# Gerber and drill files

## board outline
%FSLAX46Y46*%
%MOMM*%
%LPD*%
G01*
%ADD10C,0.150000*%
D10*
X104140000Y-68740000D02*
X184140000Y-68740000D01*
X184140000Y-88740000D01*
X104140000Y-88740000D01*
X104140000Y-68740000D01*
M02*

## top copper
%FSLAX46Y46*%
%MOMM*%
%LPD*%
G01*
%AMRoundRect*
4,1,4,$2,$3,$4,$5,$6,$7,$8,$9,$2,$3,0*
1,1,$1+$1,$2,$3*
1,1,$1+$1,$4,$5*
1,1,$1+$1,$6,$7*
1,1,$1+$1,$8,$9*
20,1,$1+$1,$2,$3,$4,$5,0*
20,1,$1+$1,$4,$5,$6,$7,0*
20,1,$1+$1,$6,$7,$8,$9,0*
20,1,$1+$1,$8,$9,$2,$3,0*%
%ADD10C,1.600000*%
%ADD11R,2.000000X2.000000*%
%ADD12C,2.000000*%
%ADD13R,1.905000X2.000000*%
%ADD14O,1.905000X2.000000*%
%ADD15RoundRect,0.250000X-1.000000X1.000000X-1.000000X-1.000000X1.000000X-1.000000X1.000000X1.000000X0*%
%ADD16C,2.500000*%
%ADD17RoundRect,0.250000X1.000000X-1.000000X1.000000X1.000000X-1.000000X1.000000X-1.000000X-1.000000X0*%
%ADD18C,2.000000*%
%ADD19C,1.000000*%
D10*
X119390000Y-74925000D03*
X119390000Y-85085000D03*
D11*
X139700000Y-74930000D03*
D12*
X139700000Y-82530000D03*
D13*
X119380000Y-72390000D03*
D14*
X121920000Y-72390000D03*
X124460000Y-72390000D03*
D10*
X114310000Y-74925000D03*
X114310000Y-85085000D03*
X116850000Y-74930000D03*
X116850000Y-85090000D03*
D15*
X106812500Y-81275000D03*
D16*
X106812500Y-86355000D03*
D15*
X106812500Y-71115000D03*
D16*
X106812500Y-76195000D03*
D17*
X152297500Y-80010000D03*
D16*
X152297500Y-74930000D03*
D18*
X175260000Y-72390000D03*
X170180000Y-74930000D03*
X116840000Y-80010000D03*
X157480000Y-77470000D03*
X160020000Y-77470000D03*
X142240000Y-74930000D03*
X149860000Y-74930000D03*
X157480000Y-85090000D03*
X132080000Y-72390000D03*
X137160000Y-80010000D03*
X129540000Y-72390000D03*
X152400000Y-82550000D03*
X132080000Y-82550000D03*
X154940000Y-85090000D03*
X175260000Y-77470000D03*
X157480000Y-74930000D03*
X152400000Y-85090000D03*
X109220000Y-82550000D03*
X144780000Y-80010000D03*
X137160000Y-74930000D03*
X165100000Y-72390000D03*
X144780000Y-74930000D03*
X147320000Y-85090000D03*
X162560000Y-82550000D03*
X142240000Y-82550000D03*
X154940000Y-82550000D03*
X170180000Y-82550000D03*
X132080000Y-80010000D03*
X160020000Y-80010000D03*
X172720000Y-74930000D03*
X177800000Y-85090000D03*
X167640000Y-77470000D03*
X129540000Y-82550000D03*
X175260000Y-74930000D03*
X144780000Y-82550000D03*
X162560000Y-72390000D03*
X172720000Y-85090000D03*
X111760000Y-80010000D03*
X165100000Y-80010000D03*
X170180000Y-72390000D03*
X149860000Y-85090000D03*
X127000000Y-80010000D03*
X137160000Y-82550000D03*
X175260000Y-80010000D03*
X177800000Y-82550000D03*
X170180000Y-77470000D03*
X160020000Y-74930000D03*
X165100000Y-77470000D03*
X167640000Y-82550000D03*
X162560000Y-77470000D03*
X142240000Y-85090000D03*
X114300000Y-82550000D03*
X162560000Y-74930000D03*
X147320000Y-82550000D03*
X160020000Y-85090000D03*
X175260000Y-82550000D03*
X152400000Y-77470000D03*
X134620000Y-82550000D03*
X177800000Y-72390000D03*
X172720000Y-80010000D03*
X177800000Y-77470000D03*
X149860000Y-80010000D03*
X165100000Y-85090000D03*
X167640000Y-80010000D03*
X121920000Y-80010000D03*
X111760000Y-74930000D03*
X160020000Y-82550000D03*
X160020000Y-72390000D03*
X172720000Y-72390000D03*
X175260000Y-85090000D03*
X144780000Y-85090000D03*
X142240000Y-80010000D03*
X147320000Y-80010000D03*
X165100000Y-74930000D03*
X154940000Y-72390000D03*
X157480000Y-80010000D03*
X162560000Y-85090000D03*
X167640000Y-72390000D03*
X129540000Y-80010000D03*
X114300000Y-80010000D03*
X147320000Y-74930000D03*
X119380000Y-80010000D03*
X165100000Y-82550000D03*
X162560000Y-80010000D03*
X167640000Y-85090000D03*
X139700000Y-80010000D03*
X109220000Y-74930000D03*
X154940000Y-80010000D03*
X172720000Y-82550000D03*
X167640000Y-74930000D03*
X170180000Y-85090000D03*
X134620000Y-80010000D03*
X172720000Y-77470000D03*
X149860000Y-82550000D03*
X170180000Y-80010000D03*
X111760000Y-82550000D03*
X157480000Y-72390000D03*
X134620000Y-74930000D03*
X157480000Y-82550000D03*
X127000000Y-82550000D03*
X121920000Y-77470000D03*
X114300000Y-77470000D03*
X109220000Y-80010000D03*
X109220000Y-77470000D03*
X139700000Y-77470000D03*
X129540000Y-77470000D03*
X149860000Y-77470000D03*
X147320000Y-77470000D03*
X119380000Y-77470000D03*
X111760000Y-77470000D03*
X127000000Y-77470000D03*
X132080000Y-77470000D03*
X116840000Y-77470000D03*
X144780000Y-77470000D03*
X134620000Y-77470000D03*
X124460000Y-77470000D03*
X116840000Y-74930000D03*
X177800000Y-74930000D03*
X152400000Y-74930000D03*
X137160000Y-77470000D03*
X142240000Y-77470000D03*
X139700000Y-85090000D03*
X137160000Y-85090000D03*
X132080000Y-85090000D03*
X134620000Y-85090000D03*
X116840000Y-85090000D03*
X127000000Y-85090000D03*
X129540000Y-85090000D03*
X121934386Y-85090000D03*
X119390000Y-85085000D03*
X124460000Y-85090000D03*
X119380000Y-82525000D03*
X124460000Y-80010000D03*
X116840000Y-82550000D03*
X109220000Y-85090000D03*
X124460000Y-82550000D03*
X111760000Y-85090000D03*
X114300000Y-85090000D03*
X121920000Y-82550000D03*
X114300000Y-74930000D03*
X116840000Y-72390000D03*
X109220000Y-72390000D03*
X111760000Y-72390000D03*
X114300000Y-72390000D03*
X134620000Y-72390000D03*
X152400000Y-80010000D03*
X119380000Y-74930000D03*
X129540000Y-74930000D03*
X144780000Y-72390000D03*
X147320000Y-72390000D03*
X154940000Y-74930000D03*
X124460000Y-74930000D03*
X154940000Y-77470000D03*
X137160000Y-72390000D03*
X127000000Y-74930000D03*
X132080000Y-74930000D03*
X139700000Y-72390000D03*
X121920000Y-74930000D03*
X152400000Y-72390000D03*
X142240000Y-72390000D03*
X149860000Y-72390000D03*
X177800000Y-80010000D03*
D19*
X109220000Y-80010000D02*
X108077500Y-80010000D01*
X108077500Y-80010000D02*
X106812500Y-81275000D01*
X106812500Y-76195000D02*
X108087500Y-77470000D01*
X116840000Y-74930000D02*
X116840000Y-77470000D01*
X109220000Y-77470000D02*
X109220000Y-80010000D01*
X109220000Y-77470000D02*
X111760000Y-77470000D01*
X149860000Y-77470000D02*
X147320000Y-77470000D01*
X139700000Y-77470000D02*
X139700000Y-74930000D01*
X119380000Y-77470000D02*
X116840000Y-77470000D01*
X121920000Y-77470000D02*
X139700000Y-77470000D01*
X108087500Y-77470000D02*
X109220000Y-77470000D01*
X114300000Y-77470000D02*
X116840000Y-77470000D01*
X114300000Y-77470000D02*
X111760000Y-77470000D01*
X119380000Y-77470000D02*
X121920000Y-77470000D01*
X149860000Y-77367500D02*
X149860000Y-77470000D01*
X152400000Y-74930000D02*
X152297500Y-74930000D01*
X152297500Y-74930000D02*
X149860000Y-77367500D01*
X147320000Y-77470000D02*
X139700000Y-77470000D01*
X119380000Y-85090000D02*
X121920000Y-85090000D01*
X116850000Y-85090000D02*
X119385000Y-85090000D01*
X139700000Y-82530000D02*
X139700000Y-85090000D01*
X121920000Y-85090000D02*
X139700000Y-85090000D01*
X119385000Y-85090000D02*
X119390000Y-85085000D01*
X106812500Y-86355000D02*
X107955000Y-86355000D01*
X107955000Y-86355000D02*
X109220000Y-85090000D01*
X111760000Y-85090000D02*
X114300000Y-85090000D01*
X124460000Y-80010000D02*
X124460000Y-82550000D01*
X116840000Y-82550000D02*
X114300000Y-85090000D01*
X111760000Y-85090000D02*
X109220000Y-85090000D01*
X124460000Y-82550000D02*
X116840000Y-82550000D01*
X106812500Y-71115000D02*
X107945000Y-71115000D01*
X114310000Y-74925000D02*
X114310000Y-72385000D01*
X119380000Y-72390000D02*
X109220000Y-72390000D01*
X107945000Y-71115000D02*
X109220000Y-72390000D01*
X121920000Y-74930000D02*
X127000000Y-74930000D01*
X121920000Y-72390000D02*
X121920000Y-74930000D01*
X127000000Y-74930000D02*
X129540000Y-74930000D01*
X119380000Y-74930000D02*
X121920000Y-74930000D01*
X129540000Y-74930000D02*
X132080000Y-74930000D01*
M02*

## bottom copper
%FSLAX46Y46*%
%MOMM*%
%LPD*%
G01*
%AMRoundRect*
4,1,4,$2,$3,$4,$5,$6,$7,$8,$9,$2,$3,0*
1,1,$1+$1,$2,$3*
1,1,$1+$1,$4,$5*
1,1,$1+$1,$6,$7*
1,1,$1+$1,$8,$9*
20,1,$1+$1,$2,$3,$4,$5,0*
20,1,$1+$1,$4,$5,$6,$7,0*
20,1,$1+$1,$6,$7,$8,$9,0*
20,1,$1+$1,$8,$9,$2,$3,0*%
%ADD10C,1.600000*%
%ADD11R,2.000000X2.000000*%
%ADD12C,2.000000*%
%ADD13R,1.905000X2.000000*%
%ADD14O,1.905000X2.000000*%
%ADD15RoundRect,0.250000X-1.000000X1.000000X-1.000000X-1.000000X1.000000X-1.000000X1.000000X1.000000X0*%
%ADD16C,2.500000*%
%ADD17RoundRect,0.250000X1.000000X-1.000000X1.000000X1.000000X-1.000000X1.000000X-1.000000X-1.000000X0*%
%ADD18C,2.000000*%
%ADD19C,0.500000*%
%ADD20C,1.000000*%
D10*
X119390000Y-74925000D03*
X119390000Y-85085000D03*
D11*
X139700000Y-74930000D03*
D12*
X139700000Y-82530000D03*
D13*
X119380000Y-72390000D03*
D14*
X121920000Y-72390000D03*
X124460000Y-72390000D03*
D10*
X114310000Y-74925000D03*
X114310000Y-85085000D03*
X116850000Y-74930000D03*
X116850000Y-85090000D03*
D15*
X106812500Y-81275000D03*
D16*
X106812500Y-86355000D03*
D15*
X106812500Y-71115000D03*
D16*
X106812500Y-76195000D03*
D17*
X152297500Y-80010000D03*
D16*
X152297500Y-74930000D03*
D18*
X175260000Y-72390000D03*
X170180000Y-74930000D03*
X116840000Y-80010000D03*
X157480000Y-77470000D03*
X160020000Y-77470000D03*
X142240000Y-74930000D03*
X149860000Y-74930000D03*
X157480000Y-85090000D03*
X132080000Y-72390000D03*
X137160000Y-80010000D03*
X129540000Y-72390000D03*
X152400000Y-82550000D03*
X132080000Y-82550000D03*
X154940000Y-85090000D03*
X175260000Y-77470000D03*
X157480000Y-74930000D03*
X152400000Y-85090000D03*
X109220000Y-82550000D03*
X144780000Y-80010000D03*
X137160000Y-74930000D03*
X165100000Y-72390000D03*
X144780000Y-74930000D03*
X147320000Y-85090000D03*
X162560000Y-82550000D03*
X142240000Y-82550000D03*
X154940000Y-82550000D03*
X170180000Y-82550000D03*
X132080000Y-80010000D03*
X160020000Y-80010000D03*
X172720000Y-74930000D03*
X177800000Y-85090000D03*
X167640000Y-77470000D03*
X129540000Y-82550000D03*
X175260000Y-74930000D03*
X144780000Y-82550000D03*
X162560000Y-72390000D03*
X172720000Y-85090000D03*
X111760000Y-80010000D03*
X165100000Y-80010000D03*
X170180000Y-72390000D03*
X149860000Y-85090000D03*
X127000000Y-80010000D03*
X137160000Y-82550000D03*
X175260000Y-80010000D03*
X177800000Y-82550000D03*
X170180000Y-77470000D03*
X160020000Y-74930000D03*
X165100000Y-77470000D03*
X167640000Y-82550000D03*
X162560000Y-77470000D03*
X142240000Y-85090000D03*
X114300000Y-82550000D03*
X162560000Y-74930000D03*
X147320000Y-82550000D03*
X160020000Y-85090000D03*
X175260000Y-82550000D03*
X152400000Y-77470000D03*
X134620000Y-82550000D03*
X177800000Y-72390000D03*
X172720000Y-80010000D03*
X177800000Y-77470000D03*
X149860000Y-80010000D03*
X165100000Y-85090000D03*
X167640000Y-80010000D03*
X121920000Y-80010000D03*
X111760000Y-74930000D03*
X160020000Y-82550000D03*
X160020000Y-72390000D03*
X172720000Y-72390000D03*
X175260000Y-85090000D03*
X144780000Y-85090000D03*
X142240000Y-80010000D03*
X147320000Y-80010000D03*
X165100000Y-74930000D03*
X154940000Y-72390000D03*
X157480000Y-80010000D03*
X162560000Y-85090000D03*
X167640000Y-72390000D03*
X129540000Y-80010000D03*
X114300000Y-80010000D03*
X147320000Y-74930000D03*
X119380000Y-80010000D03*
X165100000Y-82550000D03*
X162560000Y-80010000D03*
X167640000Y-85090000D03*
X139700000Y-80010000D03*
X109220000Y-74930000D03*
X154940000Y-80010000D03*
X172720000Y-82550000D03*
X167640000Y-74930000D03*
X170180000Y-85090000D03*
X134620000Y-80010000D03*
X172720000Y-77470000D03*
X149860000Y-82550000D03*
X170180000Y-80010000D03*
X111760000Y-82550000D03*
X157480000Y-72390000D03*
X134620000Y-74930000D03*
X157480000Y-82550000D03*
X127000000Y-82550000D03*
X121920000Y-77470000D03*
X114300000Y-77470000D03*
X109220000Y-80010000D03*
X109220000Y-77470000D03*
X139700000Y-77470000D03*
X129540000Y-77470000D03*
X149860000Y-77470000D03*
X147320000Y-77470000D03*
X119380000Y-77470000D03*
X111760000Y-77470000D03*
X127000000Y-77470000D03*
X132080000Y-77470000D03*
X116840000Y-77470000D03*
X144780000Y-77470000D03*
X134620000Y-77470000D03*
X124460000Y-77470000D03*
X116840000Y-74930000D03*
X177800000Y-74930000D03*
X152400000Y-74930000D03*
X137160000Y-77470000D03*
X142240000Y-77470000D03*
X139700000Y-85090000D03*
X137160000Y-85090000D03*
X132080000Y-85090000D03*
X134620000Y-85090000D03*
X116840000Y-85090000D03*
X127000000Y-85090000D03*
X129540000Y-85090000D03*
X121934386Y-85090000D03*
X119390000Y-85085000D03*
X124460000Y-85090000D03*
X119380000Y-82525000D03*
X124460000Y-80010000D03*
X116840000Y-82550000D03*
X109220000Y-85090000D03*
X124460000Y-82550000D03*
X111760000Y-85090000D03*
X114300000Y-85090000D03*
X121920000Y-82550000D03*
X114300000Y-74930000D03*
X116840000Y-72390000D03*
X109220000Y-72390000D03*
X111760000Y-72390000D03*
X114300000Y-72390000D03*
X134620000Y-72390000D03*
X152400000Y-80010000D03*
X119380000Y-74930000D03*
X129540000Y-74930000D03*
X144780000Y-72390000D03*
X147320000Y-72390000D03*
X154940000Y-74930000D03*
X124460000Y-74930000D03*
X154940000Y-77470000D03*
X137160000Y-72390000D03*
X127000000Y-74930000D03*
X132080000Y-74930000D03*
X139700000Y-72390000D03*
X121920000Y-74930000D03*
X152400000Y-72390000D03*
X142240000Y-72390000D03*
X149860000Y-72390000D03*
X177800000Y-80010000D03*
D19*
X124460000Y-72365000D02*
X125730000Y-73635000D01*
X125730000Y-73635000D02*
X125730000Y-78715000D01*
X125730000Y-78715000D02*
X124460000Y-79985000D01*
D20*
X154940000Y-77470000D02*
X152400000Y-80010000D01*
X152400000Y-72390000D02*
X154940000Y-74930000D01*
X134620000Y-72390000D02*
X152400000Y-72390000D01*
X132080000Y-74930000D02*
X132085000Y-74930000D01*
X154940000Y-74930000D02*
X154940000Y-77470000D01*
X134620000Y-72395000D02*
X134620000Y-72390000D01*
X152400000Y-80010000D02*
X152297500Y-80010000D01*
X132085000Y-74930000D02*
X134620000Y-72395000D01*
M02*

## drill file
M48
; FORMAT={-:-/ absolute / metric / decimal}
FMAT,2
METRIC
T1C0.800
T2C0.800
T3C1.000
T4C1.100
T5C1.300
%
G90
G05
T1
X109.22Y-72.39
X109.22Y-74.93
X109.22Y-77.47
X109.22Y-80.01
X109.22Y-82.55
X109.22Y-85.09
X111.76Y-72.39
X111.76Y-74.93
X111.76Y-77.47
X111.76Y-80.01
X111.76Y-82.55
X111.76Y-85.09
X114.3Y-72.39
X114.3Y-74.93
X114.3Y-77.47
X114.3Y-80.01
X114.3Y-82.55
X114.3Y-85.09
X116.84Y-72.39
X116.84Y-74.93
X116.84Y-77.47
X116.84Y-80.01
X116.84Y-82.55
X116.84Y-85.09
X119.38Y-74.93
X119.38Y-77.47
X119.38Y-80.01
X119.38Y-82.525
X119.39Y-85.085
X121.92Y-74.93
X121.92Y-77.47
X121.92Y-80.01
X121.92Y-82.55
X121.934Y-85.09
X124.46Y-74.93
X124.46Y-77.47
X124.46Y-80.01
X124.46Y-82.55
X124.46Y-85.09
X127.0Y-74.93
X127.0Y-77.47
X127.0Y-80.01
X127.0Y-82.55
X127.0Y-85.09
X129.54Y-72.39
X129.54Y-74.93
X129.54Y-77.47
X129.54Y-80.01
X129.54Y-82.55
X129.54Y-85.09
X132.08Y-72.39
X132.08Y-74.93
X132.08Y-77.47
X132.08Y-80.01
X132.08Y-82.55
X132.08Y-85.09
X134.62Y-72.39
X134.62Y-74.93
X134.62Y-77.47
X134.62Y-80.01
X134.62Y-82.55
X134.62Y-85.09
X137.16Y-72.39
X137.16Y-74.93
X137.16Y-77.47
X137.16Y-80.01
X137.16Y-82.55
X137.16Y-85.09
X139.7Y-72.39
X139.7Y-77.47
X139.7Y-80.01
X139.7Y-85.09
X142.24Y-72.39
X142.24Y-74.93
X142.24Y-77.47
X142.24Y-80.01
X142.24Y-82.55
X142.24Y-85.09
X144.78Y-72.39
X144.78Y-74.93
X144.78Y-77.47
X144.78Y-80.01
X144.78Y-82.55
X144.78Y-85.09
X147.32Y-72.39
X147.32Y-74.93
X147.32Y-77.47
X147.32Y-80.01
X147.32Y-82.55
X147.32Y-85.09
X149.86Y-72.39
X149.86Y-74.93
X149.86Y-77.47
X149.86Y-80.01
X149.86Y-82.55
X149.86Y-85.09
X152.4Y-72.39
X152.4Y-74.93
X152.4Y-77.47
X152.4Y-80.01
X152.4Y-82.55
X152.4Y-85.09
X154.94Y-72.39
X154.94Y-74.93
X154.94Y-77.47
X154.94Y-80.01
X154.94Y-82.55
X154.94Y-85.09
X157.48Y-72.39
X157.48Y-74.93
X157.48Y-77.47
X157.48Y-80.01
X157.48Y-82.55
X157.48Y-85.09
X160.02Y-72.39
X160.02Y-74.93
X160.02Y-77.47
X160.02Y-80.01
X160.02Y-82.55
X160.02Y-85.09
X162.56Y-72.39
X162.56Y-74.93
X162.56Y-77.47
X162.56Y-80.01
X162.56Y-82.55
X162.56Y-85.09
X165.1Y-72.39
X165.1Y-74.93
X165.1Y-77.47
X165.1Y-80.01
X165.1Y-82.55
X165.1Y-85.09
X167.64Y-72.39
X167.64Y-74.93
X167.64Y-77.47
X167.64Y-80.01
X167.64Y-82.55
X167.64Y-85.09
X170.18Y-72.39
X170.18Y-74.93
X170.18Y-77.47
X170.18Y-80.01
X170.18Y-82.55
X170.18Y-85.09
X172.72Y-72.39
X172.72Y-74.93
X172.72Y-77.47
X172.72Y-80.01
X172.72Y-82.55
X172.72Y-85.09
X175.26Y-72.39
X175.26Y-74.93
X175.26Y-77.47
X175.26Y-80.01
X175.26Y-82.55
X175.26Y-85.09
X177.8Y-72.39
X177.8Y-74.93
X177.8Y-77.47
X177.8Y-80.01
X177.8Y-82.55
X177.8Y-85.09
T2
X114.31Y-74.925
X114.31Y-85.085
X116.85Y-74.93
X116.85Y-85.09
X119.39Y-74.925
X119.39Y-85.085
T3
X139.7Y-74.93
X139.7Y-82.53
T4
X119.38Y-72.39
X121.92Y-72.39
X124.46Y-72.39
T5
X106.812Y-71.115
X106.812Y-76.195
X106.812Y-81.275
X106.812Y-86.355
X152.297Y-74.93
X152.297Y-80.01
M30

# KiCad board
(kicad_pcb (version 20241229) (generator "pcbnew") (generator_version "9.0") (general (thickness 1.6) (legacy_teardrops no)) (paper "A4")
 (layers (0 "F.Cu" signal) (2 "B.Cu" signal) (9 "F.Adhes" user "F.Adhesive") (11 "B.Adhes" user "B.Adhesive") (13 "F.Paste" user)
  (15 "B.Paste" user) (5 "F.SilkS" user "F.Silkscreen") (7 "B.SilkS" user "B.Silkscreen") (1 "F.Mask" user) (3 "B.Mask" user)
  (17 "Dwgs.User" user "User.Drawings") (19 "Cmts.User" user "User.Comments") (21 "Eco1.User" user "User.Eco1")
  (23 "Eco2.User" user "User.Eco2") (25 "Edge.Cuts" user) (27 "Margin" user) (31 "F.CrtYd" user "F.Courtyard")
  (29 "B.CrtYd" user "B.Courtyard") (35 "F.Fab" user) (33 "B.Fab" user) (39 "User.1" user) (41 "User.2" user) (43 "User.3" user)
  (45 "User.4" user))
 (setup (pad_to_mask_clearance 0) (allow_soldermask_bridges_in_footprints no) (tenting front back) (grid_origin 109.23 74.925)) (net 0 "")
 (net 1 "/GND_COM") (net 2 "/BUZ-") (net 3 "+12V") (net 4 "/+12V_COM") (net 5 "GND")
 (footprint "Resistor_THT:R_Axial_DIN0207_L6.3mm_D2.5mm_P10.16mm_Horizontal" (layer "F.Cu") (at 119.39 74.925 -90)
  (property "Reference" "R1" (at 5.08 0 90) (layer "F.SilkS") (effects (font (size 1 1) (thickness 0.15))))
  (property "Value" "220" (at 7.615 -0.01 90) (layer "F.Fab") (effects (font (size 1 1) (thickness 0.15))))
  (pad "1" thru_hole circle (at 0 0 270) (size 1.6 1.6) (drill 0.8) (layers "*.Cu" "*.Mask") (remove_unused_layers no) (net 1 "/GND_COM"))
  (pad "2" thru_hole circle (at 10.16 0 270) (size 1.6 1.6) (drill 0.8) (layers "*.Cu" "*.Mask") (remove_unused_layers no) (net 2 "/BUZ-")))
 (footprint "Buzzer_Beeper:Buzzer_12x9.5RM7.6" (layer "F.Cu") (at 139.7 74.93 -90)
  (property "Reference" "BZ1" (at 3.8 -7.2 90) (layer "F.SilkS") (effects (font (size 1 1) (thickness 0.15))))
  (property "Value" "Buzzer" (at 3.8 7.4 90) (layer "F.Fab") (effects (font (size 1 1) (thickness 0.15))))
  (pad "1" thru_hole rect (at 0 0 270) (size 2 2) (drill 1) (layers "*.Cu" "*.Mask") (remove_unused_layers no) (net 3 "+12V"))
  (pad "2" thru_hole circle (at 7.6 0 270) (size 2 2) (drill 1) (layers "*.Cu" "*.Mask") (remove_unused_layers no) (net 2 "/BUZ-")))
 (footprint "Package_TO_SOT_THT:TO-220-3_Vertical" (layer "F.Cu") (at 119.38 72.39)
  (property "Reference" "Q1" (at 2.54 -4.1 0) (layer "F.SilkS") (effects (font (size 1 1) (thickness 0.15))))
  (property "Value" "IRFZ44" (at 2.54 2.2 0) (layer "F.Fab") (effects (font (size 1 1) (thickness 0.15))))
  (pad "1" thru_hole rect (at 0 0) (size 1.905 2) (drill 1.1) (layers "*.Cu" "*.Mask") (remove_unused_layers no) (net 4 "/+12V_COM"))
  (pad "2" thru_hole oval (at 2.54 0) (size 1.905 2) (drill 1.1) (layers "*.Cu" "*.Mask") (remove_unused_layers no) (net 1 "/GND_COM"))
  (pad "3" thru_hole oval (at 5.08 0) (size 1.905 2) (drill 1.1) (layers "*.Cu" "*.Mask") (remove_unused_layers no) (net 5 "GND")))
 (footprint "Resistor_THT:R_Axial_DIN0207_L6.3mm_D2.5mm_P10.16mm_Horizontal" (layer "F.Cu") (at 114.31 74.925 -90)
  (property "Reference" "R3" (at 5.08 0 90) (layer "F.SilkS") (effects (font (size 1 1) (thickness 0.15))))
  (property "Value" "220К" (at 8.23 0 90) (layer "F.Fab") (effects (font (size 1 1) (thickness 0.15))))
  (pad "1" thru_hole circle (at 0 0 270) (size 1.6 1.6) (drill 0.8) (layers "*.Cu" "*.Mask") (remove_unused_layers no) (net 4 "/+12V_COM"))
  (pad "2" thru_hole circle (at 10.16 0 270) (size 1.6 1.6) (drill 0.8) (layers "*.Cu" "*.Mask") (remove_unused_layers no) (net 5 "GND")))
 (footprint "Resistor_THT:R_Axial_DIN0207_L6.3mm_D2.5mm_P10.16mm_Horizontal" (layer "F.Cu") (at 116.85 74.93 -90)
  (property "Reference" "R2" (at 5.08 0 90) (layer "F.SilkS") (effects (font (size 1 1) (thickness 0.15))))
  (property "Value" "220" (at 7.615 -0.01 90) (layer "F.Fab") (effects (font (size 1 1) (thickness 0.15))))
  (pad "1" thru_hole circle (at 0 0 270) (size 1.6 1.6) (drill 0.8) (layers "*.Cu" "*.Mask") (remove_unused_layers no) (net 3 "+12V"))
  (pad "2" thru_hole circle (at 10.16 0 270) (size 1.6 1.6) (drill 0.8) (layers "*.Cu" "*.Mask") (remove_unused_layers no) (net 2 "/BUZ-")))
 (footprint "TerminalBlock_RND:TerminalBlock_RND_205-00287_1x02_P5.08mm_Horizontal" (layer "F.Cu") (at 106.8125 81.275 -90)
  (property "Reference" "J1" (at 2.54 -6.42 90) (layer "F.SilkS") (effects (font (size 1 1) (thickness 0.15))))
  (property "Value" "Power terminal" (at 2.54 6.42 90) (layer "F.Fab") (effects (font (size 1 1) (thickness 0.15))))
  (pad "1" thru_hole roundrect (at 0 0 270) (size 2.5 2.5) (drill 1.3) (layers "*.Cu" "*.Mask") (remove_unused_layers no)
   (roundrect_rratio 0.1) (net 3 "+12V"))
  (pad "2" thru_hole circle (at 5.08 0 270) (size 2.5 2.5) (drill 1.3) (layers "*.Cu" "*.Mask") (remove_unused_layers no) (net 5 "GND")))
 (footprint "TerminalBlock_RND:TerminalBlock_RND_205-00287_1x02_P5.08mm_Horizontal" (layer "F.Cu") (at 106.8125 71.115 -90)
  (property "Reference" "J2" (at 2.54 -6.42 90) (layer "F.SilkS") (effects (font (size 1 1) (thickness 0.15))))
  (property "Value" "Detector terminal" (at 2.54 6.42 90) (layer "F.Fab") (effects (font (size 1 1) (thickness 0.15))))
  (pad "1" thru_hole roundrect (at 0 0 270) (size 2.5 2.5) (drill 1.3) (layers "*.Cu" "*.Mask") (remove_unused_layers no)
   (roundrect_rratio 0.1) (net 4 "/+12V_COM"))
  (pad "2" thru_hole circle (at 5.08 0 270) (size 2.5 2.5) (drill 1.3) (layers "*.Cu" "*.Mask") (remove_unused_layers no) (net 3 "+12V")))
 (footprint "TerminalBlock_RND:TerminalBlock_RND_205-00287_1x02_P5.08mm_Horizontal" (layer "F.Cu") (at 152.2975 80.01 90)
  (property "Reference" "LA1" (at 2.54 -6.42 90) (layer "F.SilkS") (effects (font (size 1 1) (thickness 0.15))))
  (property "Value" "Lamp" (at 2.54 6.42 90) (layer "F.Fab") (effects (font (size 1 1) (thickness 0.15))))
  (pad "1" thru_hole roundrect (at 0 0 90) (size 2.5 2.5) (drill 1.3) (layers "*.Cu" "*.Mask") (remove_unused_layers no)
   (roundrect_rratio 0.1) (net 1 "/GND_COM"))
  (pad "2" thru_hole circle (at 5.08 0 90) (size 2.5 2.5) (drill 1.3) (layers "*.Cu" "*.Mask") (remove_unused_layers no) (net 3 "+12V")))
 (gr_rect (start 104.14 68.74) (end 184.14 88.74) (stroke (width 0.15) (type default)) (fill no) (layer "Edge.Cuts"))
 (via (at 175.26 72.39) (size 2) (drill 0.8) (layers "F.Cu" "B.Cu") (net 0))
 (via (at 170.18 74.93) (size 2) (drill 0.8) (layers "F.Cu" "B.Cu") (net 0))
 (via (at 116.84 80.01) (size 2) (drill 0.8) (layers "F.Cu" "B.Cu") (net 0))
 (via (at 157.48 77.47) (size 2) (drill 0.8) (layers "F.Cu" "B.Cu") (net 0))
 (via (at 160.02 77.47) (size 2) (drill 0.8) (layers "F.Cu" "B.Cu") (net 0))
 (via (at 142.24 74.93) (size 2) (drill 0.8) (layers "F.Cu" "B.Cu") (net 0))
 (via (at 149.86 74.93) (size 2) (drill 0.8) (layers "F.Cu" "B.Cu") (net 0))
 (via (at 157.48 85.09) (size 2) (drill 0.8) (layers "F.Cu" "B.Cu") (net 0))
 (via (at 132.08 72.39) (size 2) (drill 0.8) (layers "F.Cu" "B.Cu") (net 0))
 (via (at 137.16 80.01) (size 2) (drill 0.8) (layers "F.Cu" "B.Cu") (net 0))
 (via (at 129.54 72.39) (size 2) (drill 0.8) (layers "F.Cu" "B.Cu") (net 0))
 (via (at 152.4 82.55) (size 2) (drill 0.8) (layers "F.Cu" "B.Cu") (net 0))
 (via (at 132.08 82.55) (size 2) (drill 0.8) (layers "F.Cu" "B.Cu") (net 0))
 (via (at 154.94 85.09) (size 2) (drill 0.8) (layers "F.Cu" "B.Cu") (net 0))
 (via (at 175.26 77.47) (size 2) (drill 0.8) (layers "F.Cu" "B.Cu") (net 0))
 (via (at 157.48 74.93) (size 2) (drill 0.8) (layers "F.Cu" "B.Cu") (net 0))
 (via (at 152.4 85.09) (size 2) (drill 0.8) (layers "F.Cu" "B.Cu") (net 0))
 (via (at 109.22 82.55) (size 2) (drill 0.8) (layers "F.Cu" "B.Cu") (free yes) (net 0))
 (via (at 144.78 80.01) (size 2) (drill 0.8) (layers "F.Cu" "B.Cu") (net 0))
 (via (at 137.16 74.93) (size 2) (drill 0.8) (layers "F.Cu" "B.Cu") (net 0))
 (via (at 165.1 72.39) (size 2) (drill 0.8) (layers "F.Cu" "B.Cu") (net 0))
 (via (at 144.78 74.93) (size 2) (drill 0.8) (layers "F.Cu" "B.Cu") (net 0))
 (via (at 147.32 85.09) (size 2) (drill 0.8) (layers "F.Cu" "B.Cu") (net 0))
 (via (at 162.56 82.55) (size 2) (drill 0.8) (layers "F.Cu" "B.Cu") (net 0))
 (via (at 142.24 82.55) (size 2) (drill 0.8) (layers "F.Cu" "B.Cu") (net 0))
 (via (at 154.94 82.55) (size 2) (drill 0.8) (layers "F.Cu" "B.Cu") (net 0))
 (via (at 170.18 82.55) (size 2) (drill 0.8) (layers "F.Cu" "B.Cu") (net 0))
 (via (at 132.08 80.01) (size 2) (drill 0.8) (layers "F.Cu" "B.Cu") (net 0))
 (via (at 160.02 80.01) (size 2) (drill 0.8) (layers "F.Cu" "B.Cu") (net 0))
 (via (at 172.72 74.93) (size 2) (drill 0.8) (layers "F.Cu" "B.Cu") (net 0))
 (via (at 177.8 85.09) (size 2) (drill 0.8) (layers "F.Cu" "B.Cu") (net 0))
 (via (at 167.64 77.47) (size 2) (drill 0.8) (layers "F.Cu" "B.Cu") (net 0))
 (via (at 129.54 82.55) (size 2) (drill 0.8) (layers "F.Cu" "B.Cu") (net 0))
 (via (at 175.26 74.93) (size 2) (drill 0.8) (layers "F.Cu" "B.Cu") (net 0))
 (via (at 144.78 82.55) (size 2) (drill 0.8) (layers "F.Cu" "B.Cu") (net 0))
 (via (at 162.56 72.39) (size 2) (drill 0.8) (layers "F.Cu" "B.Cu") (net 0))
 (via (at 172.72 85.09) (size 2) (drill 0.8) (layers "F.Cu" "B.Cu") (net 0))
 (via (at 111.76 80.01) (size 2) (drill 0.8) (layers "F.Cu" "B.Cu") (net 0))
 (via (at 165.1 80.01) (size 2) (drill 0.8) (layers "F.Cu" "B.Cu") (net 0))
 (via (at 170.18 72.39) (size 2) (drill 0.8) (layers "F.Cu" "B.Cu") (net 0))
 (via (at 149.86 85.09) (size 2) (drill 0.8) (layers "F.Cu" "B.Cu") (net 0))
 (via (at 127 80.01) (size 2) (drill 0.8) (layers "F.Cu" "B.Cu") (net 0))
 (via (at 137.16 82.55) (size 2) (drill 0.8) (layers "F.Cu" "B.Cu") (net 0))
 (via (at 175.26 80.01) (size 2) (drill 0.8) (layers "F.Cu" "B.Cu") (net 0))
 (via (at 177.8 82.55) (size 2) (drill 0.8) (layers "F.Cu" "B.Cu") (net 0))
 (via (at 170.18 77.47) (size 2) (drill 0.8) (layers "F.Cu" "B.Cu") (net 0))
 (via (at 160.02 74.93) (size 2) (drill 0.8) (layers "F.Cu" "B.Cu") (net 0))
 (via (at 165.1 77.47) (size 2) (drill 0.8) (layers "F.Cu" "B.Cu") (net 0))
 (via (at 167.64 82.55) (size 2) (drill 0.8) (layers "F.Cu" "B.Cu") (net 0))
 (via (at 162.56 77.47) (size 2) (drill 0.8) (layers "F.Cu" "B.Cu") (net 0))
 (via (at 142.24 85.09) (size 2) (drill 0.8) (layers "F.Cu" "B.Cu") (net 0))
 (via (at 114.3 82.55) (size 2) (drill 0.8) (layers "F.Cu" "B.Cu") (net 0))
 (via (at 162.56 74.93) (size 2) (drill 0.8) (layers "F.Cu" "B.Cu") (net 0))
 (via (at 147.32 82.55) (size 2) (drill 0.8) (layers "F.Cu" "B.Cu") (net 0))
 (via (at 160.02 85.09) (size 2) (drill 0.8) (layers "F.Cu" "B.Cu") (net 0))
 (via (at 175.26 82.55) (size 2) (drill 0.8) (layers "F.Cu" "B.Cu") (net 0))
 (via (at 152.4 77.47) (size 2) (drill 0.8) (layers "F.Cu" "B.Cu") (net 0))
 (via (at 134.62 82.55) (size 2) (drill 0.8) (layers "F.Cu" "B.Cu") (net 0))
 (via (at 177.8 72.39) (size 2) (drill 0.8) (layers "F.Cu" "B.Cu") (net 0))
 (via (at 172.72 80.01) (size 2) (drill 0.8) (layers "F.Cu" "B.Cu") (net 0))
 (via (at 177.8 77.47) (size 2) (drill 0.8) (layers "F.Cu" "B.Cu") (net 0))
 (via (at 149.86 80.01) (size 2) (drill 0.8) (layers "F.Cu" "B.Cu") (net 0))
 (via (at 165.1 85.09) (size 2) (drill 0.8) (layers "F.Cu" "B.Cu") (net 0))
 (via (at 167.64 80.01) (size 2) (drill 0.8) (layers "F.Cu" "B.Cu") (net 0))
 (via (at 121.92 80.01) (size 2) (drill 0.8) (layers "F.Cu" "B.Cu") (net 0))
 (via (at 111.76 74.93) (size 2) (drill 0.8) (layers "F.Cu" "B.Cu") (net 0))
 (via (at 160.02 82.55) (size 2) (drill 0.8) (layers "F.Cu" "B.Cu") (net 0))
 (via (at 160.02 72.39) (size 2) (drill 0.8) (layers "F.Cu" "B.Cu") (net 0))
 (via (at 172.72 72.39) (size 2) (drill 0.8) (layers "F.Cu" "B.Cu") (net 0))
 (via (at 175.26 85.09) (size 2) (drill 0.8) (layers "F.Cu" "B.Cu") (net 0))
 (via (at 144.78 85.09) (size 2) (drill 0.8) (layers "F.Cu" "B.Cu") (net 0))
 (via (at 142.24 80.01) (size 2) (drill 0.8) (layers "F.Cu" "B.Cu") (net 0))
 (via (at 147.32 80.01) (size 2) (drill 0.8) (layers "F.Cu" "B.Cu") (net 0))
 (via (at 165.1 74.93) (size 2) (drill 0.8) (layers "F.Cu" "B.Cu") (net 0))
 (via (at 154.94 72.39) (size 2) (drill 0.8) (layers "F.Cu" "B.Cu") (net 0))
 (via (at 157.48 80.01) (size 2) (drill 0.8) (layers "F.Cu" "B.Cu") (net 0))
 (via (at 162.56 85.09) (size 2) (drill 0.8) (layers "F.Cu" "B.Cu") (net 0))
 (via (at 167.64 72.39) (size 2) (drill 0.8) (layers "F.Cu" "B.Cu") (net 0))
 (via (at 129.54 80.01) (size 2) (drill 0.8) (layers "F.Cu" "B.Cu") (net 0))
 (via (at 114.3 80.01) (size 2) (drill 0.8) (layers "F.Cu" "B.Cu") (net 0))
 (via (at 147.32 74.93) (size 2) (drill 0.8) (layers "F.Cu" "B.Cu") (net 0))
 (via (at 119.38 80.01) (size 2) (drill 0.8) (layers "F.Cu" "B.Cu") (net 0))
 (via (at 165.1 82.55) (size 2) (drill 0.8) (layers "F.Cu" "B.Cu") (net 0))
 (via (at 162.56 80.01) (size 2) (drill 0.8) (layers "F.Cu" "B.Cu") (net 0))
 (via (at 167.64 85.09) (size 2) (drill 0.8) (layers "F.Cu" "B.Cu") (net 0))
 (via (at 139.7 80.01) (size 2) (drill 0.8) (layers "F.Cu" "B.Cu") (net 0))
 (via (at 109.22 74.93) (size 2) (drill 0.8) (layers "F.Cu" "B.Cu") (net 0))
 (via (at 154.94 80.01) (size 2) (drill 0.8) (layers "F.Cu" "B.Cu") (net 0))
 (via (at 172.72 82.55) (size 2) (drill 0.8) (layers "F.Cu" "B.Cu") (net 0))
 (via (at 167.64 74.93) (size 2) (drill 0.8) (layers "F.Cu" "B.Cu") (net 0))
 (via (at 170.18 85.09) (size 2) (drill 0.8) (layers "F.Cu" "B.Cu") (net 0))
 (via (at 134.62 80.01) (size 2) (drill 0.8) (layers "F.Cu" "B.Cu") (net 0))
 (via (at 172.72 77.47) (size 2) (drill 0.8) (layers "F.Cu" "B.Cu") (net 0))
 (via (at 149.86 82.55) (size 2) (drill 0.8) (layers "F.Cu" "B.Cu") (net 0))
 (via (at 170.18 80.01) (size 2) (drill 0.8) (layers "F.Cu" "B.Cu") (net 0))
 (via (at 111.76 82.55) (size 2) (drill 0.8) (layers "F.Cu" "B.Cu") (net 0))
 (via (at 157.48 72.39) (size 2) (drill 0.8) (layers "F.Cu" "B.Cu") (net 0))
 (via (at 134.62 74.93) (size 2) (drill 0.8) (layers "F.Cu" "B.Cu") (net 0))
 (via (at 157.48 82.55) (size 2) (drill 0.8) (layers "F.Cu" "B.Cu") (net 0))
 (via (at 127 82.55) (size 2) (drill 0.8) (layers "F.Cu" "B.Cu") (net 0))
 (segment (start 109.22 80.01) (end 108.0775 80.01) (width 1) (layer "F.Cu") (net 3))
 (segment (start 108.0775 80.01) (end 106.8125 81.275) (width 1) (layer "F.Cu") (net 3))
 (segment (start 106.8125 76.195) (end 108.0875 77.47) (width 1) (layer "F.Cu") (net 3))
 (segment (start 116.84 74.93) (end 116.84 77.47) (width 1) (layer "F.Cu") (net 3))
 (segment (start 109.22 77.47) (end 109.22 80.01) (width 1) (layer "F.Cu") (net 3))
 (segment (start 109.22 77.47) (end 111.76 77.47) (width 1) (layer "F.Cu") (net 3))
 (segment (start 149.86 77.47) (end 147.32 77.47) (width 1) (layer "F.Cu") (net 3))
 (segment (start 139.7 77.47) (end 139.7 74.93) (width 1) (layer "F.Cu") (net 3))
 (segment (start 119.38 77.47) (end 116.84 77.47) (width 1) (layer "F.Cu") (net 3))
 (segment (start 121.92 77.47) (end 139.7 77.47) (width 1) (layer "F.Cu") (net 3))
 (segment (start 108.0875 77.47) (end 109.22 77.47) (width 1) (layer "F.Cu") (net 3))
 (segment (start 114.3 77.47) (end 116.84 77.47) (width 1) (layer "F.Cu") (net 3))
 (segment (start 114.3 77.47) (end 111.76 77.47) (width 1) (layer "F.Cu") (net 3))
 (segment (start 119.38 77.47) (end 121.92 77.47) (width 1) (layer "F.Cu") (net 3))
 (segment (start 149.86 77.3675) (end 149.86 77.47) (width 1) (layer "F.Cu") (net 3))
 (segment (start 152.4 74.93) (end 152.2975 74.93) (width 1) (layer "F.Cu") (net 3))
 (segment (start 152.2975 74.93) (end 149.86 77.3675) (width 1) (layer "F.Cu") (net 3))
 (segment (start 147.32 77.47) (end 139.7 77.47) (width 1) (layer "F.Cu") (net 3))
 (via (at 121.92 77.47) (size 2) (drill 0.8) (layers "F.Cu" "B.Cu") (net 3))
 (via (at 114.3 77.47) (size 2) (drill 0.8) (layers "F.Cu" "B.Cu") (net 3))
 (via (at 109.22 80.01) (size 2) (drill 0.8) (layers "F.Cu" "B.Cu") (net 3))
 (via (at 109.22 77.47) (size 2) (drill 0.8) (layers "F.Cu" "B.Cu") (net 3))
 (via (at 139.7 77.47) (size 2) (drill 0.8) (layers "F.Cu" "B.Cu") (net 3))
 (via (at 129.54 77.47) (size 2) (drill 0.8) (layers "F.Cu" "B.Cu") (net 3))
 (via (at 149.86 77.47) (size 2) (drill 0.8) (layers "F.Cu" "B.Cu") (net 3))
 (via (at 147.32 77.47) (size 2) (drill 0.8) (layers "F.Cu" "B.Cu") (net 3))
 (via (at 119.38 77.47) (size 2) (drill 0.8) (layers "F.Cu" "B.Cu") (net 3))
 (via (at 111.76 77.47) (size 2) (drill 0.8) (layers "F.Cu" "B.Cu") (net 3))
 (via (at 127 77.47) (size 2) (drill 0.8) (layers "F.Cu" "B.Cu") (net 3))
 (via (at 132.08 77.47) (size 2) (drill 0.8) (layers "F.Cu" "B.Cu") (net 3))
 (via (at 116.84 77.47) (size 2) (drill 0.8) (layers "F.Cu" "B.Cu") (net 3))
 (via (at 144.78 77.47) (size 2) (drill 0.8) (layers "F.Cu" "B.Cu") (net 3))
 (via (at 134.62 77.47) (size 2) (drill 0.8) (layers "F.Cu" "B.Cu") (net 3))
 (via (at 124.46 77.47) (size 2) (drill 0.8) (layers "F.Cu" "B.Cu") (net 3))
 (via (at 116.84 74.93) (size 2) (drill 0.8) (layers "F.Cu" "B.Cu") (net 3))
 (via (at 177.8 74.93) (size 2) (drill 0.8) (layers "F.Cu" "B.Cu") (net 3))
 (via (at 152.4 74.93) (size 2) (drill 0.8) (layers "F.Cu" "B.Cu") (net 3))
 (via (at 137.16 77.47) (size 2) (drill 0.8) (layers "F.Cu" "B.Cu") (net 3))
 (via (at 142.24 77.47) (size 2) (drill 0.8) (layers "F.Cu" "B.Cu") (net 3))
 (segment (start 119.38 85.09) (end 121.92 85.09) (width 1) (layer "F.Cu") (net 2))
 (segment (start 116.85 85.09) (end 119.385 85.09) (width 1) (layer "F.Cu") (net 2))
 (segment (start 139.7 82.53) (end 139.7 85.09) (width 1) (layer "F.Cu") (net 2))
 (segment (start 121.92 85.09) (end 139.7 85.09) (width 1) (layer "F.Cu") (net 2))
 (segment (start 119.385 85.09) (end 119.39 85.085) (width 1) (layer "F.Cu") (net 2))
 (via (at 139.7 85.09) (size 2) (drill 0.8) (layers "F.Cu" "B.Cu") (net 2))
 (via (at 137.16 85.09) (size 2) (drill 0.8) (layers "F.Cu" "B.Cu") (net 2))
 (via (at 132.08 85.09) (size 2) (drill 0.8) (layers "F.Cu" "B.Cu") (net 2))
 (via (at 134.62 85.09) (size 2) (drill 0.8) (layers "F.Cu" "B.Cu") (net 2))
 (via (at 116.84 85.09) (size 2) (drill 0.8) (layers "F.Cu" "B.Cu") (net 2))
 (via (at 127 85.09) (size 2) (drill 0.8) (layers "F.Cu" "B.Cu") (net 2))
 (via (at 129.54 85.09) (size 2) (drill 0.8) (layers "F.Cu" "B.Cu") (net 2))
 (via (at 121.934386 85.09) (size 2) (drill 0.8) (layers "F.Cu" "B.Cu") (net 2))
 (via (at 119.39 85.085) (size 2) (drill 0.8) (layers "F.Cu" "B.Cu") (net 2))
 (via (at 124.46 85.09) (size 2) (drill 0.8) (layers "F.Cu" "B.Cu") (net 2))
 (segment (start 106.8125 86.355) (end 107.955 86.355) (width 1) (layer "F.Cu") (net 5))
 (segment (start 107.955 86.355) (end 109.22 85.09) (width 1) (layer "F.Cu") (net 5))
 (segment (start 111.76 85.09) (end 114.3 85.09) (width 1) (layer "F.Cu") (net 5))
 (segment (start 124.46 80.01) (end 124.46 82.55) (width 1) (layer "F.Cu") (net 5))
 (segment (start 116.84 82.55) (end 114.3 85.09) (width 1) (layer "F.Cu") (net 5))
 (segment (start 111.76 85.09) (end 109.22 85.09) (width 1) (layer "F.Cu") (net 5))
 (segment (start 124.46 82.55) (end 116.84 82.55) (width 1) (layer "F.Cu") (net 5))
 (via (at 119.38 82.525) (size 2) (drill 0.8) (layers "F.Cu" "B.Cu") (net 5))
 (via (at 124.46 80.01) (size 2) (drill 0.8) (layers "F.Cu" "B.Cu") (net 5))
 (via (at 116.84 82.55) (size 2) (drill 0.8) (layers "F.Cu" "B.Cu") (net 5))
 (via (at 109.22 85.09) (size 2) (drill 0.8) (layers "F.Cu" "B.Cu") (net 5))
 (via (at 124.46 82.55) (size 2) (drill 0.8) (layers "F.Cu" "B.Cu") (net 5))
 (via (at 111.76 85.09) (size 2) (drill 0.8) (layers "F.Cu" "B.Cu") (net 5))
 (via (at 114.3 85.09) (size 2) (drill 0.8) (layers "F.Cu" "B.Cu") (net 5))
 (via (at 121.92 82.55) (size 2) (drill 0.8) (layers "F.Cu" "B.Cu") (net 5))
 (segment (start 124.46 72.365) (end 125.73 73.635) (width 0.5) (layer "B.Cu") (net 5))
 (segment (start 125.73 73.635) (end 125.73 78.715) (width 0.5) (layer "B.Cu") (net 5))
 (segment (start 125.73 78.715) (end 124.46 79.985) (width 0.5) (layer "B.Cu") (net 5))
 (segment (start 106.8125 71.115) (end 107.945 71.115) (width 1) (layer "F.Cu") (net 4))
 (segment (start 114.31 74.925) (end 114.31 72.385) (width 1) (layer "F.Cu") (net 4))
 (segment (start 119.38 72.39) (end 109.22 72.39) (width 1) (layer "F.Cu") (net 4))
 (segment (start 107.945 71.115) (end 109.22 72.39) (width 1) (layer "F.Cu") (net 4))
 (via (at 114.3 74.93) (size 2) (drill 0.8) (layers "F.Cu" "B.Cu") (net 4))
 (via (at 116.84 72.39) (size 2) (drill 0.8) (layers "F.Cu" "B.Cu") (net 4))
 (via (at 109.22 72.39) (size 2) (drill 0.8) (layers "F.Cu" "B.Cu") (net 4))
 (via (at 111.76 72.39) (size 2) (drill 0.8) (layers "F.Cu" "B.Cu") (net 4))
 (via (at 114.3 72.39) (size 2) (drill 0.8) (layers "F.Cu" "B.Cu") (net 4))
 (segment (start 121.92 74.93) (end 127 74.93) (width 1) (layer "F.Cu") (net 1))
 (segment (start 121.92 72.39) (end 121.92 74.93) (width 1) (layer "F.Cu") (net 1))
 (segment (start 127 74.93) (end 129.54 74.93) (width 1) (layer "F.Cu") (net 1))
 (segment (start 119.38 74.93) (end 121.92 74.93) (width 1) (layer "F.Cu") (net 1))
 (segment (start 129.54 74.93) (end 132.08 74.93) (width 1) (layer "F.Cu") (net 1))
 (via (at 134.62 72.39) (size 2) (drill 0.8) (layers "F.Cu" "B.Cu") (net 1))
 (via (at 152.4 80.01) (size 2) (drill 0.8) (layers "F.Cu" "B.Cu") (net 1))
 (via (at 119.38 74.93) (size 2) (drill 0.8) (layers "F.Cu" "B.Cu") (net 1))
 (via (at 129.54 74.93) (size 2) (drill 0.8) (layers "F.Cu" "B.Cu") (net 1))
 (via (at 144.78 72.39) (size 2) (drill 0.8) (layers "F.Cu" "B.Cu") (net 1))
 (via (at 147.32 72.39) (size 2) (drill 0.8) (layers "F.Cu" "B.Cu") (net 1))
 (via (at 154.94 74.93) (size 2) (drill 0.8) (layers "F.Cu" "B.Cu") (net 1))
 (via (at 124.46 74.93) (size 2) (drill 0.8) (layers "F.Cu" "B.Cu") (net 1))
 (via (at 154.94 77.47) (size 2) (drill 0.8) (layers "F.Cu" "B.Cu") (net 1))
 (via (at 137.16 72.39) (size 2) (drill 0.8) (layers "F.Cu" "B.Cu") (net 1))
 (via (at 127 74.93) (size 2) (drill 0.8) (layers "F.Cu" "B.Cu") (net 1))
 (via (at 132.08 74.93) (size 2) (drill 0.8) (layers "F.Cu" "B.Cu") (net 1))
 (via (at 139.7 72.39) (size 2) (drill 0.8) (layers "F.Cu" "B.Cu") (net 1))
 (via (at 121.92 74.93) (size 2) (drill 0.8) (layers "F.Cu" "B.Cu") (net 1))
 (via (at 152.4 72.39) (size 2) (drill 0.8) (layers "F.Cu" "B.Cu") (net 1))
 (via (at 142.24 72.39) (size 2) (drill 0.8) (layers "F.Cu" "B.Cu") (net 1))
 (via (at 149.86 72.39) (size 2) (drill 0.8) (layers "F.Cu" "B.Cu") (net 1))
 (via (at 177.8 80.01) (size 2) (drill 0.8) (layers "F.Cu" "B.Cu") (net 1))
 (segment (start 154.94 77.47) (end 152.4 80.01) (width 1) (layer "B.Cu") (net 1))
 (segment (start 152.4 72.39) (end 154.94 74.93) (width 1) (layer "B.Cu") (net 1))
 (segment (start 134.62 72.39) (end 152.4 72.39) (width 1) (layer "B.Cu") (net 1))
 (segment (start 132.08 74.93) (end 132.085 74.93) (width 1) (layer "B.Cu") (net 1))
 (segment (start 154.94 74.93) (end 154.94 77.47) (width 1) (layer "B.Cu") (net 1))
 (segment (start 134.62 72.395) (end 134.62 72.39) (width 1) (layer "B.Cu") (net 1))
 (segment (start 152.4 80.01) (end 152.2975 80.01) (width 1) (layer "B.Cu") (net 1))
 (segment (start 132.085 74.93) (end 134.62 72.395) (width 1) (layer "B.Cu") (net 1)))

